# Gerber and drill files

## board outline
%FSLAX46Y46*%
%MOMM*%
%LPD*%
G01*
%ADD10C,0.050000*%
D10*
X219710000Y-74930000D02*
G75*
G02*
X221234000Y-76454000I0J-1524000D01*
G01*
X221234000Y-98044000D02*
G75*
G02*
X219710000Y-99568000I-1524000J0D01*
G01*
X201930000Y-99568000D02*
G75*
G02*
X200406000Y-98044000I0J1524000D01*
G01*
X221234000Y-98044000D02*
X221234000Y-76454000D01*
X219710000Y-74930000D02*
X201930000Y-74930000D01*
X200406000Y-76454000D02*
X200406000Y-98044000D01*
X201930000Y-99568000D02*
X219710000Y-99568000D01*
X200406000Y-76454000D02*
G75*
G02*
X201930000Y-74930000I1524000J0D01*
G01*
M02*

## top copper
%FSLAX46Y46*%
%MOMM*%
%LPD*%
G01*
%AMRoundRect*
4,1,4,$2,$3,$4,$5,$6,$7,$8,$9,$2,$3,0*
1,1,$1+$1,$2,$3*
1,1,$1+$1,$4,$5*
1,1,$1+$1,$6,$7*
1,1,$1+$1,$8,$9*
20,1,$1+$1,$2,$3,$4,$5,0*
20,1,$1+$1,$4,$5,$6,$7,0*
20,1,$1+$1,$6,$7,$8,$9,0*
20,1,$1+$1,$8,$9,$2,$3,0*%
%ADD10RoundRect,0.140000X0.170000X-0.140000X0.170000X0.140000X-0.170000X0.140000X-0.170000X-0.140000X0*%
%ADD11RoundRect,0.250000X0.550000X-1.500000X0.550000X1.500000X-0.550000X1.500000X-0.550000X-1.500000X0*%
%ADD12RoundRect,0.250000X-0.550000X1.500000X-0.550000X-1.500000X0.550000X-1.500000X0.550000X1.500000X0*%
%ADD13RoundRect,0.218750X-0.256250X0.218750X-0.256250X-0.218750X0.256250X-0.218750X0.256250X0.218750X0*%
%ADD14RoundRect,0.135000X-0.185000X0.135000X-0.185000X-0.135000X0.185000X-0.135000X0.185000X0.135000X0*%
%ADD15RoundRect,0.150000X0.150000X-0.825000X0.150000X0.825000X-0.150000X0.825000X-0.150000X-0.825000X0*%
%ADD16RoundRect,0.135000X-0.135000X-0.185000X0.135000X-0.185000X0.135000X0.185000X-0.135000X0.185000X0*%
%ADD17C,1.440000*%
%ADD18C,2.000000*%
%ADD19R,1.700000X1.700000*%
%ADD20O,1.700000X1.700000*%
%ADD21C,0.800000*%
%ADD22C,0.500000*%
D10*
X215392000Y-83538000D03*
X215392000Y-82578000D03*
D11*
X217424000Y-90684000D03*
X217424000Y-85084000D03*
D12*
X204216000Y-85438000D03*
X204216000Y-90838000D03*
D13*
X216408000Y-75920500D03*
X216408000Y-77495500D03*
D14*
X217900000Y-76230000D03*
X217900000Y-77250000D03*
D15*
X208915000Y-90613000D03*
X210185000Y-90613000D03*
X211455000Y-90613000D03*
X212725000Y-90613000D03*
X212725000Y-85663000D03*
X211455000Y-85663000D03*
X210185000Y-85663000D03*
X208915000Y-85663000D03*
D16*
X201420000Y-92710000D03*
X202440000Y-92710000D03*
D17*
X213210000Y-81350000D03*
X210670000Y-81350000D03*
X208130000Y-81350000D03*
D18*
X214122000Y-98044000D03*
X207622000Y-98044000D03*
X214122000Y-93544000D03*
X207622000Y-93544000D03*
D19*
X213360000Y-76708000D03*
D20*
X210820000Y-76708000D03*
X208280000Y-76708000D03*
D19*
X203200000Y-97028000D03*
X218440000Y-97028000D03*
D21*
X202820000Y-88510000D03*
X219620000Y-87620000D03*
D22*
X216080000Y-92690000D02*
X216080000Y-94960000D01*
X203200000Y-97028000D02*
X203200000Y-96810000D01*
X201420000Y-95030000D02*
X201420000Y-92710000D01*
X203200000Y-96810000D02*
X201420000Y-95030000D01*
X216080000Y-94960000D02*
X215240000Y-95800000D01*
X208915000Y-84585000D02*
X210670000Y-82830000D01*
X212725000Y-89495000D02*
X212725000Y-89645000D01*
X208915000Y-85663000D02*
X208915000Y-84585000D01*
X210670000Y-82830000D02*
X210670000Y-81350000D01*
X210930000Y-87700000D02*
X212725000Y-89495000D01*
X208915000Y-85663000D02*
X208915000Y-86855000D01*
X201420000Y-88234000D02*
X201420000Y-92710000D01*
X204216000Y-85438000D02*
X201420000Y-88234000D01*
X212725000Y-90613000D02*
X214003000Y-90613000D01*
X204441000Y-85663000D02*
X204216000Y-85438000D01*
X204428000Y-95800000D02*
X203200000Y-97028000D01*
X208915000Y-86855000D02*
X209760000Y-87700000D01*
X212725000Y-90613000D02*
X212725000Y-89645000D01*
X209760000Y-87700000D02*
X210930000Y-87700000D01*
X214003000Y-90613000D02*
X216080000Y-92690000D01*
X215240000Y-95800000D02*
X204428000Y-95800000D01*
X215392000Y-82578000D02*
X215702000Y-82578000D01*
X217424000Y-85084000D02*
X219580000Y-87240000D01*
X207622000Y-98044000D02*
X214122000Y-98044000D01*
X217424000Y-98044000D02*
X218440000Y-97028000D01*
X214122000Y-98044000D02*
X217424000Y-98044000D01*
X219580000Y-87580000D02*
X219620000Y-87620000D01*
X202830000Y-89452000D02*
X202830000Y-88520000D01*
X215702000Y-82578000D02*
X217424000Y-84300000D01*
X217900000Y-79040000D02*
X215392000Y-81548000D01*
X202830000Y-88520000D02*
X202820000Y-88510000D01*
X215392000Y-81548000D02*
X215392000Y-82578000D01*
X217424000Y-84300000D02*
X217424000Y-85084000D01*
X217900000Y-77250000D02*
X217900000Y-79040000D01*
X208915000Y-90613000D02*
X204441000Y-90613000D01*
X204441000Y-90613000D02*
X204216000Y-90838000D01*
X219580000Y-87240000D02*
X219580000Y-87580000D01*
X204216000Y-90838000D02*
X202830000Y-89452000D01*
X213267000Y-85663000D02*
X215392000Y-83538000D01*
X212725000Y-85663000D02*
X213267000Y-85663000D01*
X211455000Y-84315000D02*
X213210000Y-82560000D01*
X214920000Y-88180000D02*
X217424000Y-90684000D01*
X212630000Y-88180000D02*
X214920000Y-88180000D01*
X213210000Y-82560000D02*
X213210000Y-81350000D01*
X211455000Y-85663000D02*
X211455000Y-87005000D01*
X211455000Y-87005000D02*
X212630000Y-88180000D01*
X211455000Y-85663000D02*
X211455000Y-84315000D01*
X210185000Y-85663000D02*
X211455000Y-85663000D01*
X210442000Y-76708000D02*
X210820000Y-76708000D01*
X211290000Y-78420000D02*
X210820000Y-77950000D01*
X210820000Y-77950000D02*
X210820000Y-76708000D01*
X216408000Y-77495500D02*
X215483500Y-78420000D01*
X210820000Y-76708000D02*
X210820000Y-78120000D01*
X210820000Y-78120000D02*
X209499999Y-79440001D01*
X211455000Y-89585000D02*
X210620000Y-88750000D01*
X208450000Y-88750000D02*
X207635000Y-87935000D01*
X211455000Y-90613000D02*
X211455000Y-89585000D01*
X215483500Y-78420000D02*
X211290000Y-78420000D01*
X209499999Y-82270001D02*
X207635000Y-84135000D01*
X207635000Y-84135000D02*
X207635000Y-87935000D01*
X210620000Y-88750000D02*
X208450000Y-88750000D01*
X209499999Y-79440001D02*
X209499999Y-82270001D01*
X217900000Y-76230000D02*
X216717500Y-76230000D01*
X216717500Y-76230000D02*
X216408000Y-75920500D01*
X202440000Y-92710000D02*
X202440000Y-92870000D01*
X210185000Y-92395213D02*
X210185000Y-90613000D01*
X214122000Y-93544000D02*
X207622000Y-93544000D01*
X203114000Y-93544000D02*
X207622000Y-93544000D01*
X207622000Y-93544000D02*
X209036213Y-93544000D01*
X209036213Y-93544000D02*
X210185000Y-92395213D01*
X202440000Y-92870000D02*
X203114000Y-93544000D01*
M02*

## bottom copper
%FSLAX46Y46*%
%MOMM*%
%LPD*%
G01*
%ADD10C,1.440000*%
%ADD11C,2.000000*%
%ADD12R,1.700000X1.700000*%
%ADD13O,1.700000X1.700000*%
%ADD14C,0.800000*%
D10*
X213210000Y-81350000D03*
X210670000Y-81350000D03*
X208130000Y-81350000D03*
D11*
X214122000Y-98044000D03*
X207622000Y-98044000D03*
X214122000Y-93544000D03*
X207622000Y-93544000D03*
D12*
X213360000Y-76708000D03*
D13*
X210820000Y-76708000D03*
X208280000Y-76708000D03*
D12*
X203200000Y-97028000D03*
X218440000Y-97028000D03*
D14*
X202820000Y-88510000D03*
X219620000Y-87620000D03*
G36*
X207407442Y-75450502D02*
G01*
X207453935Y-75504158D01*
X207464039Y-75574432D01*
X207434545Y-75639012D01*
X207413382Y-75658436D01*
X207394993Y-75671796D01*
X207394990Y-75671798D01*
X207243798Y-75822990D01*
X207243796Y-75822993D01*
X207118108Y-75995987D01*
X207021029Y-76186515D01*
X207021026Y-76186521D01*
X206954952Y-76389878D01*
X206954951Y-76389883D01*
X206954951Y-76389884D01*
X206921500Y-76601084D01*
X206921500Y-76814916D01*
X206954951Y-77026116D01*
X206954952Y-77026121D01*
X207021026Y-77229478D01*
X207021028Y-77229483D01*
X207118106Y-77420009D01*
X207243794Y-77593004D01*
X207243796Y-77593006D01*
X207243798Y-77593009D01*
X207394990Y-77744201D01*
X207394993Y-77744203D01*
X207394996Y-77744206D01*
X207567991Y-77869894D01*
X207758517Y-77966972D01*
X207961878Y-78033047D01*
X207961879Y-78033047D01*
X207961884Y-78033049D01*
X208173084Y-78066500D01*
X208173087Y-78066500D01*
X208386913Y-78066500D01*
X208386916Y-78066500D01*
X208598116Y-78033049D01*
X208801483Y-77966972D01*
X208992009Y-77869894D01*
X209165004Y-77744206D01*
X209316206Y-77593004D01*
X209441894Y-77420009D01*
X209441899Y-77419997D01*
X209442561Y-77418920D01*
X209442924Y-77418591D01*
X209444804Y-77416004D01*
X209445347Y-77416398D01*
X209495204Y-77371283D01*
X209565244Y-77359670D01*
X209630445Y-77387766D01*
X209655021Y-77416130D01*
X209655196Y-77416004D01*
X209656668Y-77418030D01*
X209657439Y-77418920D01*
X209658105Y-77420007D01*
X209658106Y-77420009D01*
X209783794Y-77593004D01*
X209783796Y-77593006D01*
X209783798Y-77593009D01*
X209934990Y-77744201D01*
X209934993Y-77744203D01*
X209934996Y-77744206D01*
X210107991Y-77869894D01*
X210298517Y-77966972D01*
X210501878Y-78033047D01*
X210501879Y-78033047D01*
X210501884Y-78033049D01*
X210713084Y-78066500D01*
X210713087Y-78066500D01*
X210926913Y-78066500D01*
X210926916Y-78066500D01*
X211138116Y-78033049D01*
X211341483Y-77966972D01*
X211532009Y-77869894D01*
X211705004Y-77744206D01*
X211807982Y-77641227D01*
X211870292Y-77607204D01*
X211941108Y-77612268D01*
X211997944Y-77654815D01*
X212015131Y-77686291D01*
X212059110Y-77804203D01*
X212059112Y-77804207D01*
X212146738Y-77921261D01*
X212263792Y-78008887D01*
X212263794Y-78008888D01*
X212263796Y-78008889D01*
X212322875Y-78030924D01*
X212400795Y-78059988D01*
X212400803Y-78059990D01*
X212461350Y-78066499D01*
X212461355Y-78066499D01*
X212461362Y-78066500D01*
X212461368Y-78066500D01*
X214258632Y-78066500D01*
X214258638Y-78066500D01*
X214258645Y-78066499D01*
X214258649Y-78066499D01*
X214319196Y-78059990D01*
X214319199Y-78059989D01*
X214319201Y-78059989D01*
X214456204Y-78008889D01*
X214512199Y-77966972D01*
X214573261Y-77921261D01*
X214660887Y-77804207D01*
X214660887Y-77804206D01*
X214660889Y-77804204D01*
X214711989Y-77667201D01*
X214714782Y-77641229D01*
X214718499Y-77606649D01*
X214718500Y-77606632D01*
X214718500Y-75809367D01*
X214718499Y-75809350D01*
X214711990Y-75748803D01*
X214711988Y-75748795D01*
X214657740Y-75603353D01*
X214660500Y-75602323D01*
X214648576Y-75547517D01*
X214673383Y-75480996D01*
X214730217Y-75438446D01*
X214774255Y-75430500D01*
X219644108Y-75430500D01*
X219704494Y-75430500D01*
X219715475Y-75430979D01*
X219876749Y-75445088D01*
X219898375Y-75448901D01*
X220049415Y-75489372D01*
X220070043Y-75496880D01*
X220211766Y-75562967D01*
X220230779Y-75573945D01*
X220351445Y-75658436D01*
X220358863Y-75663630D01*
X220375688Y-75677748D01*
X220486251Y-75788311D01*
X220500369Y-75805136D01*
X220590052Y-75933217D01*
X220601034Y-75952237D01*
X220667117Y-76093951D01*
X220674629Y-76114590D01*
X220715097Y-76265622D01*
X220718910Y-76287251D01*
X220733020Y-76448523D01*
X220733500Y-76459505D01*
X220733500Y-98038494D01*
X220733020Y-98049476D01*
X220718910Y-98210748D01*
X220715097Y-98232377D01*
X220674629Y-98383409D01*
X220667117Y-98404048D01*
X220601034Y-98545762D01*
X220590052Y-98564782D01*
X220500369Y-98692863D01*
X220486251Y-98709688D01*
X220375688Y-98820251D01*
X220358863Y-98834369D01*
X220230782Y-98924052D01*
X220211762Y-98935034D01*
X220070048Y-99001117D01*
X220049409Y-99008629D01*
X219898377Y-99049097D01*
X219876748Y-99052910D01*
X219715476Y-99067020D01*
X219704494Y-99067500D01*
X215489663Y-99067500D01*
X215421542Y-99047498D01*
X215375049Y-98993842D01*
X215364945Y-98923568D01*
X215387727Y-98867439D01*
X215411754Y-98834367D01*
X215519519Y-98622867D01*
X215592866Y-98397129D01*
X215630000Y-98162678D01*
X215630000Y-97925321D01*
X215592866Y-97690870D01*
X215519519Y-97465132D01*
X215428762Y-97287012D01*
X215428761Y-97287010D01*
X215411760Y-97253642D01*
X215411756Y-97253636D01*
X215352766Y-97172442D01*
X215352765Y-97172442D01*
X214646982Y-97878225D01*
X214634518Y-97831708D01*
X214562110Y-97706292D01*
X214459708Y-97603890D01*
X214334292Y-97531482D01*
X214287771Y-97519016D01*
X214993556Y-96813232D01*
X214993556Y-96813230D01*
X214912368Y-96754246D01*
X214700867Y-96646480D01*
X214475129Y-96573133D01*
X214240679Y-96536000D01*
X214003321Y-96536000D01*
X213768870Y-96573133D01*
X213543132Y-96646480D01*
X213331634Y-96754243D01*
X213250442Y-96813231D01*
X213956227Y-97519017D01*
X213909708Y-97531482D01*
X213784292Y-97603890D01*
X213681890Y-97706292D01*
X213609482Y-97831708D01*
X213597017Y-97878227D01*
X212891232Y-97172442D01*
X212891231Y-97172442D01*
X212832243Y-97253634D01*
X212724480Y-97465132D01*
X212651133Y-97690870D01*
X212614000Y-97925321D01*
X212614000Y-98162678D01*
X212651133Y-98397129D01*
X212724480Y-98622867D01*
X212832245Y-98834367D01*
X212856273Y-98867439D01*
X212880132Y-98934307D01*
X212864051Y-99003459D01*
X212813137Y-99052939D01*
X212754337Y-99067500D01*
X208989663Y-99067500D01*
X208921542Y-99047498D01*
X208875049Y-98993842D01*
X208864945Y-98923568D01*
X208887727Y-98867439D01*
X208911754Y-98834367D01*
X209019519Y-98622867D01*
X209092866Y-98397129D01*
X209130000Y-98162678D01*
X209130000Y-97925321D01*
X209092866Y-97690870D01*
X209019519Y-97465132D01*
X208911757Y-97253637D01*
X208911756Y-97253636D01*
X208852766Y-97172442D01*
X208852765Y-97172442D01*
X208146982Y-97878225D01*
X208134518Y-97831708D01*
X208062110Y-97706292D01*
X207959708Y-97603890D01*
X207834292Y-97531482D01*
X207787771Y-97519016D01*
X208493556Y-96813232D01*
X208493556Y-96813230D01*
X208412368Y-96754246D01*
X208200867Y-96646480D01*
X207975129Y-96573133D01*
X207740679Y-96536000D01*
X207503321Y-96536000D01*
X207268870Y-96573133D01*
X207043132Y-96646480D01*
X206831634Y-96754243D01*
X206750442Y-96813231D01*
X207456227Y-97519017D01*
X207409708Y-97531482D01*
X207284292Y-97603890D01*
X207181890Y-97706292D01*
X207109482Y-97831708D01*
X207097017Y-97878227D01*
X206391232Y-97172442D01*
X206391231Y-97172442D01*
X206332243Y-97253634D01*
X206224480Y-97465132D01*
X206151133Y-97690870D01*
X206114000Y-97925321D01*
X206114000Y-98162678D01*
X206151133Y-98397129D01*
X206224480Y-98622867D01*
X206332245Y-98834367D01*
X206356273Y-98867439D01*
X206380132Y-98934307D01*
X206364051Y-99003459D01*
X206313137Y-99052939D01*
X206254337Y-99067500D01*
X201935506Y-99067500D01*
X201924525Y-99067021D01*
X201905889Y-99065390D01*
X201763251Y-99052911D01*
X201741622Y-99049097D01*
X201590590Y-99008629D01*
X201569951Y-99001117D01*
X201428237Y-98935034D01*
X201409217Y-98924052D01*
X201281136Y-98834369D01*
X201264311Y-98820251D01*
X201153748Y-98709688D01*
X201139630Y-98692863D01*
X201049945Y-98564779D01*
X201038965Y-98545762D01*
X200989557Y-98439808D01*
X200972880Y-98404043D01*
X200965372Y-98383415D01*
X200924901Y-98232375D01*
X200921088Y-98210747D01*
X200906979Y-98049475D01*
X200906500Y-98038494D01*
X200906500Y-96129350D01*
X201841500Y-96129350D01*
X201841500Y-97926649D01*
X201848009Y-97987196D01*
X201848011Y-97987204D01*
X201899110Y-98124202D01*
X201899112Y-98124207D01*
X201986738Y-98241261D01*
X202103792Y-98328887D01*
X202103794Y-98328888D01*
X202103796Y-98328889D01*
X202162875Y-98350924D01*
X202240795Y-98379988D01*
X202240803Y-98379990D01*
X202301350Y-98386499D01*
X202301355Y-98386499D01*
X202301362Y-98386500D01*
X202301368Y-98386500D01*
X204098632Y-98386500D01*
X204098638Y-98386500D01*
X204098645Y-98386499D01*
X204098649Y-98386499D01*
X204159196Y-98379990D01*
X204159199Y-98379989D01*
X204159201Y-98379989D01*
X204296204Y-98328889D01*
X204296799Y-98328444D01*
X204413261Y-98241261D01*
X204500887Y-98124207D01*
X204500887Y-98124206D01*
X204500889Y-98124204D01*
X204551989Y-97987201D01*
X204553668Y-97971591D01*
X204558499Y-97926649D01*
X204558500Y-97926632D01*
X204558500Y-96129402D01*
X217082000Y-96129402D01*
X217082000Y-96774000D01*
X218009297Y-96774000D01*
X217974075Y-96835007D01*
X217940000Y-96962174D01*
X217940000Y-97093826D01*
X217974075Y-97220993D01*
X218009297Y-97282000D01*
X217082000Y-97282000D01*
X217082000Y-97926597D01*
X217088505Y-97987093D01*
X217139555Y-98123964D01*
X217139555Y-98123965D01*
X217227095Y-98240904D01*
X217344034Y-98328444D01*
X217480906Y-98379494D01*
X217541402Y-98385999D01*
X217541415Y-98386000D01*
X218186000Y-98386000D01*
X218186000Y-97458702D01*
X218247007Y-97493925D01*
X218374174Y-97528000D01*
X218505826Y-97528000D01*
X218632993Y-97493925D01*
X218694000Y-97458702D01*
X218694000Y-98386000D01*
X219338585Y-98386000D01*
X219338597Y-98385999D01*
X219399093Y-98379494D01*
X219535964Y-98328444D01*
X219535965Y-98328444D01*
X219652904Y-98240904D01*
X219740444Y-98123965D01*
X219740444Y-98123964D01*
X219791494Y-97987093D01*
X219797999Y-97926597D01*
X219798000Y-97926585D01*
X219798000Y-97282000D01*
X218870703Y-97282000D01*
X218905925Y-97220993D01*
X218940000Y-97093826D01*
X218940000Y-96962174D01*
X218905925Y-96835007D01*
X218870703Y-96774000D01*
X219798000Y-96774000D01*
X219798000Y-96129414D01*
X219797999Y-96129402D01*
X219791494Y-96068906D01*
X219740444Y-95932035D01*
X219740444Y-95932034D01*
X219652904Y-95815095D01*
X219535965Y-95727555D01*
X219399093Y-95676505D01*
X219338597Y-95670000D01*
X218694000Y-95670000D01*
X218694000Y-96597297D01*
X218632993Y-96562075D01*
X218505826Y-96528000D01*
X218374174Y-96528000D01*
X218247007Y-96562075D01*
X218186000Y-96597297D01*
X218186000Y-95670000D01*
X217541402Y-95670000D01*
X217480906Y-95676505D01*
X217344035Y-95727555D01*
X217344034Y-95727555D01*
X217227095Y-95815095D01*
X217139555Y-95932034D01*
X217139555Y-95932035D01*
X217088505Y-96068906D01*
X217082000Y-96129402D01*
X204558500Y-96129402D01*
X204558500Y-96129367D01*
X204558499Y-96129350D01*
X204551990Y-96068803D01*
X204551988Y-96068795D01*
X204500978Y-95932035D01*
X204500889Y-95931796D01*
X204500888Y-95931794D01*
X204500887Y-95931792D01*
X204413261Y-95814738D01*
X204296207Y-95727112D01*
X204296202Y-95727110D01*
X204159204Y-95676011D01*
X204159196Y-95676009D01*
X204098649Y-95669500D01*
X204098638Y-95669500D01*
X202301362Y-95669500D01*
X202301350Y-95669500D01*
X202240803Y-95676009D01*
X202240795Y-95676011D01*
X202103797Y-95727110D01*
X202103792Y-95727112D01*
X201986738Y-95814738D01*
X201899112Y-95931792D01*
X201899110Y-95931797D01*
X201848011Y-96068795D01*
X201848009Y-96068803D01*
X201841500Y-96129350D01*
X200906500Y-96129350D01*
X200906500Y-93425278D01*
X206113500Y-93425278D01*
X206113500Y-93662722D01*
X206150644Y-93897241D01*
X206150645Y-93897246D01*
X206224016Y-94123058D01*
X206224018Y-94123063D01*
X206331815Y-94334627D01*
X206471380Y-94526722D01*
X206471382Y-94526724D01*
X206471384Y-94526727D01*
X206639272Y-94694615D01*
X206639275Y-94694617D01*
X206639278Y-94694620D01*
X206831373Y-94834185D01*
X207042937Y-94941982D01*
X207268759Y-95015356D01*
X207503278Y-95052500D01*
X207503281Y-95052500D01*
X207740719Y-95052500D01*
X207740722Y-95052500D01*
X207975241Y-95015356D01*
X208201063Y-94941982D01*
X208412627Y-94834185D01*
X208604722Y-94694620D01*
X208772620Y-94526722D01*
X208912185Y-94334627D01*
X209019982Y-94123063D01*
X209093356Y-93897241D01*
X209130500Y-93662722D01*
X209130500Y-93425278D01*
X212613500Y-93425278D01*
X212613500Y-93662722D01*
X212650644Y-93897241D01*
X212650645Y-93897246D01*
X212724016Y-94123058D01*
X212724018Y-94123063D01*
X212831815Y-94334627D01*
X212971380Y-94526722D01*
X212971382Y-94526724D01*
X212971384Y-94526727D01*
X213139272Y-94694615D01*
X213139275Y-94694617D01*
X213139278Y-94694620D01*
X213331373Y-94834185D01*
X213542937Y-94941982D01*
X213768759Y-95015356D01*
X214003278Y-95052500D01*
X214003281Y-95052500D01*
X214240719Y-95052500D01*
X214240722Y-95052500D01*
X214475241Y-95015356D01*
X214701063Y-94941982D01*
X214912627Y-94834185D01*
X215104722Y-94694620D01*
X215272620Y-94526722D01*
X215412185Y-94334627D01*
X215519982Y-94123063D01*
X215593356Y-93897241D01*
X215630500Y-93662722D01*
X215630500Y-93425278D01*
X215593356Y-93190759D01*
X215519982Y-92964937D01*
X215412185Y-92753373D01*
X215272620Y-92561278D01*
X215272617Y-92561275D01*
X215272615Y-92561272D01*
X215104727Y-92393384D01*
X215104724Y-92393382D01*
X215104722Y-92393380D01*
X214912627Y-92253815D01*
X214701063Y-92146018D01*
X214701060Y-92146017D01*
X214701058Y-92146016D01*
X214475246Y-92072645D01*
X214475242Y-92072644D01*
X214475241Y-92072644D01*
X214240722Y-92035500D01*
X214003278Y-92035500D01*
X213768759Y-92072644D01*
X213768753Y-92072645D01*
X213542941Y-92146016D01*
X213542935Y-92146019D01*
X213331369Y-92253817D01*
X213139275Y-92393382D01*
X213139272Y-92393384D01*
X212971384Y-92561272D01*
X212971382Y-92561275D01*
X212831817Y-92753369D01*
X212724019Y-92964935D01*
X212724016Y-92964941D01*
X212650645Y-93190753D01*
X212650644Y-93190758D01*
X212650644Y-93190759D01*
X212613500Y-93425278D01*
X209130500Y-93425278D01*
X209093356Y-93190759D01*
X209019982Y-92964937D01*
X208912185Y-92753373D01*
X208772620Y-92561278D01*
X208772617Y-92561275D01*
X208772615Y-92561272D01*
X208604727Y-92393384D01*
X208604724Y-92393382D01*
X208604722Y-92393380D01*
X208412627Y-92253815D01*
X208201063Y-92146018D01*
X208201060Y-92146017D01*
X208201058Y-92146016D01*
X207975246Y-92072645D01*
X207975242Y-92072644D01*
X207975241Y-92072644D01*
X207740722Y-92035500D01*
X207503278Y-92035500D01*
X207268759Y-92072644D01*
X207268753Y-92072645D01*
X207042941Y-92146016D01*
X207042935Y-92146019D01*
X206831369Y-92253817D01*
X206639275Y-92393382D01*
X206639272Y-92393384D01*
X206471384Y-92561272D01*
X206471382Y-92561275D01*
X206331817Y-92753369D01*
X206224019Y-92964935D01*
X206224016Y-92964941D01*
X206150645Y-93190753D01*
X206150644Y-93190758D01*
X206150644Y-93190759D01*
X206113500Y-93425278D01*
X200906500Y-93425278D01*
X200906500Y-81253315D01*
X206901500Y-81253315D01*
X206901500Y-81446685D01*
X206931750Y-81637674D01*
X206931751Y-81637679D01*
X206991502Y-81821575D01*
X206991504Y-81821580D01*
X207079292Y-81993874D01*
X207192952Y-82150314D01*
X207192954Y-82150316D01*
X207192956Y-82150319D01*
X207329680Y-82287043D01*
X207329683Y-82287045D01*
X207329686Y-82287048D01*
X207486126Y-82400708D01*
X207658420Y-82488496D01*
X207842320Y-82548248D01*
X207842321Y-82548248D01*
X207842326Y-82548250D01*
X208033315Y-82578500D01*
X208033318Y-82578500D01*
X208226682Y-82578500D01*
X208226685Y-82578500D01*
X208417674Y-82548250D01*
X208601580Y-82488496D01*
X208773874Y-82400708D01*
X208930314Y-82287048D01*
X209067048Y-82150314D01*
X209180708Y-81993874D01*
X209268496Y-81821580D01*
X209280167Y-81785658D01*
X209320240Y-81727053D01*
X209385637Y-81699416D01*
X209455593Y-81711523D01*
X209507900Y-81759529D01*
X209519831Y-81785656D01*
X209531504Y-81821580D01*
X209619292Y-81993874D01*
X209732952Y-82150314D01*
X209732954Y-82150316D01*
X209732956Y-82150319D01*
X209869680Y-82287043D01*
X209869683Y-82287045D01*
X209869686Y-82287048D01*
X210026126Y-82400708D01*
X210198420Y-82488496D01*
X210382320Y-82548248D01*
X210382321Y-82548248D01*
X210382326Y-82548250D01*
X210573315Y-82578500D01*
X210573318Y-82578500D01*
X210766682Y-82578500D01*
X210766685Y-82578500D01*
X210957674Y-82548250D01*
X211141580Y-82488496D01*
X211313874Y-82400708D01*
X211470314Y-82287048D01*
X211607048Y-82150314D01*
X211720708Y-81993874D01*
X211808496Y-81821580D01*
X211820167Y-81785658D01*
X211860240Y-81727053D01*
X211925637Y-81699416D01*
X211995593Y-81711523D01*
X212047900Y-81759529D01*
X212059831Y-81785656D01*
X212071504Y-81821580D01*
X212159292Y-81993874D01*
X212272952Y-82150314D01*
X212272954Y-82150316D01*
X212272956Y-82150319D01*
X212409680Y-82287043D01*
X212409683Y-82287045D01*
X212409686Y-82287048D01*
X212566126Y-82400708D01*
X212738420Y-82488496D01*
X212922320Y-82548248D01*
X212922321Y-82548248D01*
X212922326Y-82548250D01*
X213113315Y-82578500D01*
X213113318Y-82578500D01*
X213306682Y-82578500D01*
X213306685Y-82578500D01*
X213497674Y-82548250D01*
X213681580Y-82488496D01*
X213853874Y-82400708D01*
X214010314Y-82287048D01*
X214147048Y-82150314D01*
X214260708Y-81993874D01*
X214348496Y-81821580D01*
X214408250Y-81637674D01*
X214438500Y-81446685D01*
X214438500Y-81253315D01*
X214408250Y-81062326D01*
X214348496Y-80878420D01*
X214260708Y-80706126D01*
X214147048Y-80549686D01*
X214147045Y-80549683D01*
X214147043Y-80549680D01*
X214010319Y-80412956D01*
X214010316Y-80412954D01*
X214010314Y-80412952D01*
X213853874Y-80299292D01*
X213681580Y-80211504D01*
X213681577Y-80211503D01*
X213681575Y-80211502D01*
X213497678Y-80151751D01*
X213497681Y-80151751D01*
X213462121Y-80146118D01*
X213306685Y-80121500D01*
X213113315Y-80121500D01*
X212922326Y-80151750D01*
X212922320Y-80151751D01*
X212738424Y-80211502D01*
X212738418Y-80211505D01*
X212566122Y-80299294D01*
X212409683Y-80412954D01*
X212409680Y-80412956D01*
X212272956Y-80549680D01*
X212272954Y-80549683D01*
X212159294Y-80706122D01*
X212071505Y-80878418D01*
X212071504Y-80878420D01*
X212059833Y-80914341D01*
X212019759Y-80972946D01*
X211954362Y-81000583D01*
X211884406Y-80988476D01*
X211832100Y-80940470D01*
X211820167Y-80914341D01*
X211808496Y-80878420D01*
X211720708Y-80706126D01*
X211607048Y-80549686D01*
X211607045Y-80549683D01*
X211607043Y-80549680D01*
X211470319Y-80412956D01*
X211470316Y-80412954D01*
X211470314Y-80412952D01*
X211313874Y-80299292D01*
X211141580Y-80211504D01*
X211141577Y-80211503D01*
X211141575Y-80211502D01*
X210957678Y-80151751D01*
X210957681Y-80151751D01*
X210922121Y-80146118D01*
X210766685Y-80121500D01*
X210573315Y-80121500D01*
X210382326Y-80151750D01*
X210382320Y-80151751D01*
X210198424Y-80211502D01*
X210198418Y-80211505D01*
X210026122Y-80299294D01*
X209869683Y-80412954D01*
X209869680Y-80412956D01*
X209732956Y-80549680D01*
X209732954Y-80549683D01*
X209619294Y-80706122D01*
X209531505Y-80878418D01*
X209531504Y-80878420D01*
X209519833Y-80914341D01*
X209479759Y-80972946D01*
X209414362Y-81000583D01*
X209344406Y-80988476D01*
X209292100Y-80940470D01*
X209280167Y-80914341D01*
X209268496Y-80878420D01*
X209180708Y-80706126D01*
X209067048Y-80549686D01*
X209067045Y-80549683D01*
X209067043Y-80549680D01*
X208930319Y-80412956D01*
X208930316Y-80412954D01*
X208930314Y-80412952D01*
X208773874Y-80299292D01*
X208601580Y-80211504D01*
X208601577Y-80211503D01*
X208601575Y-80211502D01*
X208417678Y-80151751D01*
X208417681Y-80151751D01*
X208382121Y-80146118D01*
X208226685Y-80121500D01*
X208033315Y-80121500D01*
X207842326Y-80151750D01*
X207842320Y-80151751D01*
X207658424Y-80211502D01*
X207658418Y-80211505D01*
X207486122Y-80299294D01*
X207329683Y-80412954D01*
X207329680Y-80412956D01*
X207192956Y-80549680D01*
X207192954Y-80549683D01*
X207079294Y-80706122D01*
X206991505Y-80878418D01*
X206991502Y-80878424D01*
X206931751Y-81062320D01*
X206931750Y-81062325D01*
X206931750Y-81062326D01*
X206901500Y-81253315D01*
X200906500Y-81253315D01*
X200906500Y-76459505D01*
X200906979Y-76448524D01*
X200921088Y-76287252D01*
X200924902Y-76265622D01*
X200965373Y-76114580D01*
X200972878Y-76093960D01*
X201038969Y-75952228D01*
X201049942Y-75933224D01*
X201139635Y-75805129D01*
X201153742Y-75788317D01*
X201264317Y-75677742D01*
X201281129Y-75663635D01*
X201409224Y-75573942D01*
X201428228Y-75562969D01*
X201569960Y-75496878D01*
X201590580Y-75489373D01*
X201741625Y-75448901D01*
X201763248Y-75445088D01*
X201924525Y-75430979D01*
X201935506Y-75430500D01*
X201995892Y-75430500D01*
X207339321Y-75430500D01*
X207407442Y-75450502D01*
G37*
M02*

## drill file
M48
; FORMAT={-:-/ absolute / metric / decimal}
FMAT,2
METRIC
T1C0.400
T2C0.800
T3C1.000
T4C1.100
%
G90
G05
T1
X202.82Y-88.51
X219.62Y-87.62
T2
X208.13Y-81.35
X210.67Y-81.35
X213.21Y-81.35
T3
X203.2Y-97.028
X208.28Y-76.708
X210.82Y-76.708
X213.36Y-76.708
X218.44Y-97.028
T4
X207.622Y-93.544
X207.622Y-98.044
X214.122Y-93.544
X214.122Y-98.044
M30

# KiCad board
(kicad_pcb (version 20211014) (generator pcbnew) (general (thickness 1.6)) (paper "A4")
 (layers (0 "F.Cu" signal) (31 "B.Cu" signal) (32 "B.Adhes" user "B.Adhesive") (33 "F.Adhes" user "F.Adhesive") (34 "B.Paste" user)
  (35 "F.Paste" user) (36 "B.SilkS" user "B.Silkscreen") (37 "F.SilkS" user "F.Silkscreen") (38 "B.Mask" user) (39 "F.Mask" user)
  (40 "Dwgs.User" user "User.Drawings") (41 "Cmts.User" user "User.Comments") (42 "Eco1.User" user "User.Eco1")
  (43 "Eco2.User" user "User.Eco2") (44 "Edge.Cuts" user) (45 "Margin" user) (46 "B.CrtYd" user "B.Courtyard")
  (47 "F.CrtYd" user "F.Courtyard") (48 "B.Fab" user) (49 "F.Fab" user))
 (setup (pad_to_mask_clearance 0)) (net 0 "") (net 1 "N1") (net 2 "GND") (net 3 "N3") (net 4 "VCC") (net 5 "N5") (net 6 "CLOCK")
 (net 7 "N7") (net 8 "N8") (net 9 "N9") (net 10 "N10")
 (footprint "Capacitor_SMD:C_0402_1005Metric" (layer "F.Cu") (at 215.392 83.058 90)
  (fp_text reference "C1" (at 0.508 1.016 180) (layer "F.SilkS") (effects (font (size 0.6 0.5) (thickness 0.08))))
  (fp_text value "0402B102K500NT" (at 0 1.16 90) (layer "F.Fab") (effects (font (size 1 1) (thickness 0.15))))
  (pad "1" smd roundrect locked (at -0.48 0 90) (size 0.56 0.62) (layers "F.Cu" "F.Paste" "F.Mask") (roundrect_rratio 0.25) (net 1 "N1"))
  (pad "2" smd roundrect locked (at 0.48 0 90) (size 0.56 0.62) (layers "F.Cu" "F.Paste" "F.Mask") (roundrect_rratio 0.25) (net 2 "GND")))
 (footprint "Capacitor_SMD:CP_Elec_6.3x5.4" (layer "F.Cu") (at 217.424 87.884 90)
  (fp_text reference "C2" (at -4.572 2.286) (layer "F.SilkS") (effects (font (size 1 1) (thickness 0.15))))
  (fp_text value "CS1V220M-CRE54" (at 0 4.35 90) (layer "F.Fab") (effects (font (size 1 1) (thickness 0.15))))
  (pad "1" smd roundrect locked (at -2.8 0 90) (size 3.5 1.6) (layers "F.Cu" "F.Paste" "F.Mask") (roundrect_rratio 0.15625) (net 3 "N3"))
  (pad "2" smd roundrect locked (at 2.8 0 90) (size 3.5 1.6) (layers "F.Cu" "F.Paste" "F.Mask") (roundrect_rratio 0.15625) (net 2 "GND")))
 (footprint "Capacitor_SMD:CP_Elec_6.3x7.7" (layer "F.Cu") (at 204.216 88.138 -90)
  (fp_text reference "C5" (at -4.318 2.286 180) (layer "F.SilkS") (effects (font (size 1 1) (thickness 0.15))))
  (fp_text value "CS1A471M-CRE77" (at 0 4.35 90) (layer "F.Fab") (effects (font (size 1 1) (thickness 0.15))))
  (pad "1" smd roundrect locked (at -2.7 0 270) (size 3.5 1.6) (layers "F.Cu" "F.Paste" "F.Mask") (roundrect_rratio 0.15625) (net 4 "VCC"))
  (pad "2" smd roundrect locked (at 2.7 0 270) (size 3.5 1.6) (layers "F.Cu" "F.Paste" "F.Mask") (roundrect_rratio 0.15625) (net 2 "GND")))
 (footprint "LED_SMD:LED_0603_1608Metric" (layer "F.Cu") (at 216.408 76.708 -90)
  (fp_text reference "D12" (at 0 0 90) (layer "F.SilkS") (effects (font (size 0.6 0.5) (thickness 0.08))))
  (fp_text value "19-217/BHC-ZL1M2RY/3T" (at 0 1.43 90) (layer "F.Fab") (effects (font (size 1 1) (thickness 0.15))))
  (pad "1" smd roundrect locked (at -0.7875 0 270) (size 0.875 0.95) (layers "F.Cu" "F.Paste" "F.Mask") (roundrect_rratio 0.25) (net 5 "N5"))
  (pad "2" smd roundrect locked (at 0.7875 0 270) (size 0.875 0.95) (layers "F.Cu" "F.Paste" "F.Mask") (roundrect_rratio 0.25)
   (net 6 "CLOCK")))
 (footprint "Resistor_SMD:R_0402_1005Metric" (layer "F.Cu") (at 217.9 76.74 -90)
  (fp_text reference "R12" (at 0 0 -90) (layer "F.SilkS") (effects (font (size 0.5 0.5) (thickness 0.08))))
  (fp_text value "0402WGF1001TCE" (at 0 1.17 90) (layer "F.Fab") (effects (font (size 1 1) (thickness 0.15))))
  (pad "1" smd roundrect locked (at -0.51 0 270) (size 0.54 0.64) (layers "F.Cu" "F.Paste" "F.Mask") (roundrect_rratio 0.25) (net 5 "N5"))
  (pad "2" smd roundrect locked (at 0.51 0 270) (size 0.54 0.64) (layers "F.Cu" "F.Paste" "F.Mask") (roundrect_rratio 0.25) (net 2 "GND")))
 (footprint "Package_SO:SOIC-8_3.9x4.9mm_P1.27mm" (layer "F.Cu") (at 210.82 88.138 90)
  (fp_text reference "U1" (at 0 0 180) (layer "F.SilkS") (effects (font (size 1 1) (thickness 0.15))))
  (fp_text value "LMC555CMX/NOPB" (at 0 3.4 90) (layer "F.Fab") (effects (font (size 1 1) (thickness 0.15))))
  (pad "1" smd roundrect locked (at -2.475 -1.905 90) (size 1.95 0.6) (layers "F.Cu" "F.Paste" "F.Mask") (roundrect_rratio 0.25)
   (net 2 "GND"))
  (pad "2" smd roundrect locked (at -2.475 -0.635 90) (size 1.95 0.6) (layers "F.Cu" "F.Paste" "F.Mask") (roundrect_rratio 0.25)
   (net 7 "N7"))
  (pad "3" smd roundrect locked (at -2.475 0.635 90) (size 1.95 0.6) (layers "F.Cu" "F.Paste" "F.Mask") (roundrect_rratio 0.25)
   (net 6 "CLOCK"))
  (pad "4" smd roundrect locked (at -2.475 1.905 90) (size 1.95 0.6) (layers "F.Cu" "F.Paste" "F.Mask") (roundrect_rratio 0.25)
   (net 4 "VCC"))
  (pad "5" smd roundrect locked (at 2.475 1.905 90) (size 1.95 0.6) (layers "F.Cu" "F.Paste" "F.Mask") (roundrect_rratio 0.25) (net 1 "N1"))
  (pad "6" smd roundrect locked (at 2.475 0.635 90) (size 1.95 0.6) (layers "F.Cu" "F.Paste" "F.Mask") (roundrect_rratio 0.25) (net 3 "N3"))
  (pad "7" smd roundrect locked (at 2.475 -0.635 90) (size 1.95 0.6) (layers "F.Cu" "F.Paste" "F.Mask") (roundrect_rratio 0.25) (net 3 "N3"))
  (pad "8" smd roundrect locked (at 2.475 -1.905 90) (size 1.95 0.6) (layers "F.Cu" "F.Paste" "F.Mask") (roundrect_rratio 0.25)
   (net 4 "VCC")))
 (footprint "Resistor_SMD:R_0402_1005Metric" (layer "F.Cu") (at 201.93 92.71)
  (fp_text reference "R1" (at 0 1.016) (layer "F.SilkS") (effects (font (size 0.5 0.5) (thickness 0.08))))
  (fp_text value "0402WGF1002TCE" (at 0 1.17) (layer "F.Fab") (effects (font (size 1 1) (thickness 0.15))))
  (pad "1" smd roundrect locked (at -0.51 0) (size 0.54 0.64) (layers "F.Cu" "F.Paste" "F.Mask") (roundrect_rratio 0.25) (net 4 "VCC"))
  (pad "2" smd roundrect locked (at 0.51 0) (size 0.54 0.64) (layers "F.Cu" "F.Paste" "F.Mask") (roundrect_rratio 0.25) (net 7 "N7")))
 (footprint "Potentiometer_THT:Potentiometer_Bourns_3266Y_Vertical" (layer "F.Cu") (at 213.21 81.35)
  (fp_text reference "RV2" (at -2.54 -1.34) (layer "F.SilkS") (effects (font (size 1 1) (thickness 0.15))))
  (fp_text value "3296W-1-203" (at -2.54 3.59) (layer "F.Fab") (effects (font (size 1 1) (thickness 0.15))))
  (pad "1" thru_hole circle locked (at 0 0) (size 1.44 1.44) (drill 0.8) (layers *.Cu *.Mask) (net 3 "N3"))
  (pad "2" thru_hole circle locked (at -2.54 0) (size 1.44 1.44) (drill 0.8) (layers *.Cu *.Mask) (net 4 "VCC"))
  (pad "3" thru_hole circle locked (at -5.08 0) (size 1.44 1.44) (drill 0.8) (layers *.Cu *.Mask) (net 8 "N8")))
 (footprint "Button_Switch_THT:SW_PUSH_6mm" (layer "F.Cu") (at 214.122 98.044 180)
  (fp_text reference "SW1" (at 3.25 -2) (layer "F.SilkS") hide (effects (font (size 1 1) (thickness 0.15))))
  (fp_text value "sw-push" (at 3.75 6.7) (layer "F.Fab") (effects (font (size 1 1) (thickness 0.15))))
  (pad "1" thru_hole circle locked (at 0 0 270) (size 2 2) (drill 1.1) (layers *.Cu *.Mask) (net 2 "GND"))
  (pad "1" thru_hole circle locked (at 6.5 0 270) (size 2 2) (drill 1.1) (layers *.Cu *.Mask) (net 2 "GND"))
  (pad "2" thru_hole circle locked (at 0 4.5 270) (size 2 2) (drill 1.1) (layers *.Cu *.Mask) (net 7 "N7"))
  (pad "2" thru_hole circle locked (at 6.5 4.5 270) (size 2 2) (drill 1.1) (layers *.Cu *.Mask) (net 7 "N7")))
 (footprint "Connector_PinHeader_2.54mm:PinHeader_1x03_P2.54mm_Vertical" (layer "B.Cu") (at 213.36 76.708 90)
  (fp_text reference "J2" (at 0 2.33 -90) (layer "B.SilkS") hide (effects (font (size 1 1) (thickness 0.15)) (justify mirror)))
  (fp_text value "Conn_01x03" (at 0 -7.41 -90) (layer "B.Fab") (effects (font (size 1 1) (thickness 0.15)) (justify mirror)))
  (pad "1" thru_hole rect locked (at 0 0 90) (size 1.7 1.7) (drill 1) (layers *.Cu *.Mask) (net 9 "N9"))
  (pad "2" thru_hole oval locked (at 0 -2.54 90) (size 1.7 1.7) (drill 1) (layers *.Cu *.Mask) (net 6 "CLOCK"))
  (pad "3" thru_hole oval locked (at 0 -5.08 90) (size 1.7 1.7) (drill 1) (layers *.Cu *.Mask) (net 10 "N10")))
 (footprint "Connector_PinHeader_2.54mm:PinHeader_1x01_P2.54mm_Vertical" (layer "B.Cu") (at 203.2 97.028)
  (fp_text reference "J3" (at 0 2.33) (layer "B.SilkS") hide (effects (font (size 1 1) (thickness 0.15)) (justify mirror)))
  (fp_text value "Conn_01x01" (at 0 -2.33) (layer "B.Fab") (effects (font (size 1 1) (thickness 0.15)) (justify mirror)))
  (pad "1" thru_hole rect locked (at 0 0) (size 1.7 1.7) (drill 1) (layers *.Cu *.Mask) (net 4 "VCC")))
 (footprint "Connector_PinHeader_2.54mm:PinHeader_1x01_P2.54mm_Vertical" (layer "B.Cu") (at 218.44 97.028)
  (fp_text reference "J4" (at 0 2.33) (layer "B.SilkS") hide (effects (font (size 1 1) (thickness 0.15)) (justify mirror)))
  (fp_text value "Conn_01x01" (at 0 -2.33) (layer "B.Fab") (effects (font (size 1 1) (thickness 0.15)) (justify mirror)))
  (pad "1" thru_hole rect locked (at 0 0) (size 1.7 1.7) (drill 1) (layers *.Cu *.Mask) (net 2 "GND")))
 (gr_arc (start 219.71 74.93) (mid 220.787631 75.376369) (end 221.234 76.454) (layer "Edge.Cuts") (width 0.05))
 (gr_arc (start 221.234 98.044) (mid 220.787631 99.121631) (end 219.71 99.568) (layer "Edge.Cuts") (width 0.05))
 (gr_arc (start 201.93 99.568) (mid 200.852369 99.121631) (end 200.406 98.044) (layer "Edge.Cuts") (width 0.05))
 (gr_line (start 221.234 98.044) (end 221.234 76.454) (layer "Edge.Cuts") (width 0.05))
 (gr_line (start 219.71 74.93) (end 201.93 74.93) (layer "Edge.Cuts") (width 0.05))
 (gr_line (start 200.406 76.454) (end 200.406 98.044) (layer "Edge.Cuts") (width 0.05))
 (gr_line (start 201.93 99.568) (end 219.71 99.568) (layer "Edge.Cuts") (width 0.05))
 (gr_arc (start 200.406 76.454) (mid 200.852369 75.376369) (end 201.93 74.93) (layer "Edge.Cuts") (width 0.05))
 (segment (start 216.08 92.69) (end 216.08 94.96) (width 0.5) (layer "F.Cu") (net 4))
 (segment (start 203.2 97.028) (end 203.2 96.81) (width 0.5) (layer "F.Cu") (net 4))
 (segment (start 201.42 95.03) (end 201.42 92.71) (width 0.5) (layer "F.Cu") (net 4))
 (segment (start 203.2 96.81) (end 201.42 95.03) (width 0.5) (layer "F.Cu") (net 4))
 (segment (start 216.08 94.96) (end 215.24 95.8) (width 0.5) (layer "F.Cu") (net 4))
 (segment (start 208.915 84.585) (end 210.67 82.83) (width 0.5) (layer "F.Cu") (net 4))
 (segment (start 212.725 89.495) (end 212.725 89.645) (width 0.5) (layer "F.Cu") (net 4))
 (segment (start 208.915 85.663) (end 208.915 84.585) (width 0.5) (layer "F.Cu") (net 4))
 (segment (start 210.67 82.83) (end 210.67 81.35) (width 0.5) (layer "F.Cu") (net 4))
 (segment (start 210.93 87.7) (end 212.725 89.495) (width 0.5) (layer "F.Cu") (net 4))
 (segment (start 208.915 85.663) (end 208.915 86.855) (width 0.5) (layer "F.Cu") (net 4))
 (segment (start 201.42 88.234) (end 201.42 92.71) (width 0.5) (layer "F.Cu") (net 4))
 (segment (start 204.216 85.438) (end 201.42 88.234) (width 0.5) (layer "F.Cu") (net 4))
 (segment (start 212.725 90.613) (end 214.003 90.613) (width 0.5) (layer "F.Cu") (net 4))
 (segment (start 204.441 85.663) (end 204.216 85.438) (width 0.5) (layer "F.Cu") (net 4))
 (segment (start 204.428 95.8) (end 203.2 97.028) (width 0.5) (layer "F.Cu") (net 4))
 (segment (start 208.915 86.855) (end 209.76 87.7) (width 0.5) (layer "F.Cu") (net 4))
 (segment (start 212.725 90.613) (end 212.725 89.645) (width 0.5) (layer "F.Cu") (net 4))
 (segment (start 209.76 87.7) (end 210.93 87.7) (width 0.5) (layer "F.Cu") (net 4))
 (segment (start 214.003 90.613) (end 216.08 92.69) (width 0.5) (layer "F.Cu") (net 4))
 (segment (start 215.24 95.8) (end 204.428 95.8) (width 0.5) (layer "F.Cu") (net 4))
 (segment (start 215.392 82.578) (end 215.702 82.578) (width 0.5) (layer "F.Cu") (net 2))
 (segment (start 217.424 85.084) (end 219.58 87.24) (width 0.5) (layer "F.Cu") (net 2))
 (segment (start 207.622 98.044) (end 214.122 98.044) (width 0.5) (layer "F.Cu") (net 2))
 (segment (start 217.424 98.044) (end 218.44 97.028) (width 0.5) (layer "F.Cu") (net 2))
 (segment (start 214.122 98.044) (end 217.424 98.044) (width 0.5) (layer "F.Cu") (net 2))
 (segment (start 219.58 87.58) (end 219.62 87.62) (width 0.5) (layer "F.Cu") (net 2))
 (segment (start 202.83 89.452) (end 202.83 88.52) (width 0.5) (layer "F.Cu") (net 2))
 (segment (start 215.702 82.578) (end 217.424 84.3) (width 0.5) (layer "F.Cu") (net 2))
 (segment (start 217.9 79.04) (end 215.392 81.548) (width 0.5) (layer "F.Cu") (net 2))
 (segment (start 202.83 88.52) (end 202.82 88.51) (width 0.5) (layer "F.Cu") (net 2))
 (segment (start 215.392 81.548) (end 215.392 82.578) (width 0.5) (layer "F.Cu") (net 2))
 (segment (start 217.424 84.3) (end 217.424 85.084) (width 0.5) (layer "F.Cu") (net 2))
 (segment (start 217.9 77.25) (end 217.9 79.04) (width 0.5) (layer "F.Cu") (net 2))
 (segment (start 208.915 90.613) (end 204.441 90.613) (width 0.5) (layer "F.Cu") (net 2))
 (segment (start 204.441 90.613) (end 204.216 90.838) (width 0.5) (layer "F.Cu") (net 2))
 (segment (start 219.58 87.24) (end 219.58 87.58) (width 0.5) (layer "F.Cu") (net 2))
 (segment (start 204.216 90.838) (end 202.83 89.452) (width 0.5) (layer "F.Cu") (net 2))
 (via (at 202.82 88.51) (size 0.8) (drill 0.4) (layers "F.Cu" "B.Cu") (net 2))
 (via (at 219.62 87.62) (size 0.8) (drill 0.4) (layers "F.Cu" "B.Cu") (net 2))
 (segment (start 213.267 85.663) (end 215.392 83.538) (width 0.5) (layer "F.Cu") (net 1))
 (segment (start 212.725 85.663) (end 213.267 85.663) (width 0.5) (layer "F.Cu") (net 1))
 (segment (start 211.455 84.315) (end 213.21 82.56) (width 0.5) (layer "F.Cu") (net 3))
 (segment (start 214.92 88.18) (end 217.424 90.684) (width 0.5) (layer "F.Cu") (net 3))
 (segment (start 212.63 88.18) (end 214.92 88.18) (width 0.5) (layer "F.Cu") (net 3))
 (segment (start 213.21 82.56) (end 213.21 81.35) (width 0.5) (layer "F.Cu") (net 3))
 (segment (start 211.455 85.663) (end 211.455 87.005) (width 0.5) (layer "F.Cu") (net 3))
 (segment (start 211.455 87.005) (end 212.63 88.18) (width 0.5) (layer "F.Cu") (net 3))
 (segment (start 211.455 85.663) (end 211.455 84.315) (width 0.5) (layer "F.Cu") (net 3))
 (segment (start 210.185 85.663) (end 211.455 85.663) (width 0.5) (layer "F.Cu") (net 3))
 (segment (start 210.442 76.708) (end 210.82 76.708) (width 0.5) (layer "F.Cu") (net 6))
 (segment (start 211.29 78.42) (end 210.82 77.95) (width 0.5) (layer "F.Cu") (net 6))
 (segment (start 210.82 77.95) (end 210.82 76.708) (width 0.5) (layer "F.Cu") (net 6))
 (segment (start 216.408 77.4955) (end 215.4835 78.42) (width 0.5) (layer "F.Cu") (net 6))
 (segment (start 210.82 76.708) (end 210.82 78.12) (width 0.5) (layer "F.Cu") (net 6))
 (segment (start 210.82 78.12) (end 209.499999 79.440001) (width 0.5) (layer "F.Cu") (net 6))
 (segment (start 211.455 89.585) (end 210.62 88.75) (width 0.5) (layer "F.Cu") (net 6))
 (segment (start 208.45 88.75) (end 207.635 87.935) (width 0.5) (layer "F.Cu") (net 6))
 (segment (start 211.455 90.613) (end 211.455 89.585) (width 0.5) (layer "F.Cu") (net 6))
 (segment (start 215.4835 78.42) (end 211.29 78.42) (width 0.5) (layer "F.Cu") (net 6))
 (segment (start 209.499999 82.270001) (end 207.635 84.135) (width 0.5) (layer "F.Cu") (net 6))
 (segment (start 207.635 84.135) (end 207.635 87.935) (width 0.5) (layer "F.Cu") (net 6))
 (segment (start 210.62 88.75) (end 208.45 88.75) (width 0.5) (layer "F.Cu") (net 6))
 (segment (start 209.499999 79.440001) (end 209.499999 82.270001) (width 0.5) (layer "F.Cu") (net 6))
 (segment (start 217.9 76.23) (end 216.7175 76.23) (width 0.5) (layer "F.Cu") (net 5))
 (segment (start 216.7175 76.23) (end 216.408 75.9205) (width 0.5) (layer "F.Cu") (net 5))
 (segment (start 202.44 92.71) (end 202.44 92.87) (width 0.5) (layer "F.Cu") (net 7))
 (segment (start 210.185 92.395213) (end 210.185 90.613) (width 0.5) (layer "F.Cu") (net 7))
 (segment (start 214.122 93.544) (end 207.622 93.544) (width 0.5) (layer "F.Cu") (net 7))
 (segment (start 203.114 93.544) (end 207.622 93.544) (width 0.5) (layer "F.Cu") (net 7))
 (segment (start 207.622 93.544) (end 209.036213 93.544) (width 0.5) (layer "F.Cu") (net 7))
 (segment (start 209.036213 93.544) (end 210.185 92.395213) (width 0.5) (layer "F.Cu") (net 7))
 (segment (start 202.44 92.87) (end 203.114 93.544) (width 0.5) (layer "F.Cu") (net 7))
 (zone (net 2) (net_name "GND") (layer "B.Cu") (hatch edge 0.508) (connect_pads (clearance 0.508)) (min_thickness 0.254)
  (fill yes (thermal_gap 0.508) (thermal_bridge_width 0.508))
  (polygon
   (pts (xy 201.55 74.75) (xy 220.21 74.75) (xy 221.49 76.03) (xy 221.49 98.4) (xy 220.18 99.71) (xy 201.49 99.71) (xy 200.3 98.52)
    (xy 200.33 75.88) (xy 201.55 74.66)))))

